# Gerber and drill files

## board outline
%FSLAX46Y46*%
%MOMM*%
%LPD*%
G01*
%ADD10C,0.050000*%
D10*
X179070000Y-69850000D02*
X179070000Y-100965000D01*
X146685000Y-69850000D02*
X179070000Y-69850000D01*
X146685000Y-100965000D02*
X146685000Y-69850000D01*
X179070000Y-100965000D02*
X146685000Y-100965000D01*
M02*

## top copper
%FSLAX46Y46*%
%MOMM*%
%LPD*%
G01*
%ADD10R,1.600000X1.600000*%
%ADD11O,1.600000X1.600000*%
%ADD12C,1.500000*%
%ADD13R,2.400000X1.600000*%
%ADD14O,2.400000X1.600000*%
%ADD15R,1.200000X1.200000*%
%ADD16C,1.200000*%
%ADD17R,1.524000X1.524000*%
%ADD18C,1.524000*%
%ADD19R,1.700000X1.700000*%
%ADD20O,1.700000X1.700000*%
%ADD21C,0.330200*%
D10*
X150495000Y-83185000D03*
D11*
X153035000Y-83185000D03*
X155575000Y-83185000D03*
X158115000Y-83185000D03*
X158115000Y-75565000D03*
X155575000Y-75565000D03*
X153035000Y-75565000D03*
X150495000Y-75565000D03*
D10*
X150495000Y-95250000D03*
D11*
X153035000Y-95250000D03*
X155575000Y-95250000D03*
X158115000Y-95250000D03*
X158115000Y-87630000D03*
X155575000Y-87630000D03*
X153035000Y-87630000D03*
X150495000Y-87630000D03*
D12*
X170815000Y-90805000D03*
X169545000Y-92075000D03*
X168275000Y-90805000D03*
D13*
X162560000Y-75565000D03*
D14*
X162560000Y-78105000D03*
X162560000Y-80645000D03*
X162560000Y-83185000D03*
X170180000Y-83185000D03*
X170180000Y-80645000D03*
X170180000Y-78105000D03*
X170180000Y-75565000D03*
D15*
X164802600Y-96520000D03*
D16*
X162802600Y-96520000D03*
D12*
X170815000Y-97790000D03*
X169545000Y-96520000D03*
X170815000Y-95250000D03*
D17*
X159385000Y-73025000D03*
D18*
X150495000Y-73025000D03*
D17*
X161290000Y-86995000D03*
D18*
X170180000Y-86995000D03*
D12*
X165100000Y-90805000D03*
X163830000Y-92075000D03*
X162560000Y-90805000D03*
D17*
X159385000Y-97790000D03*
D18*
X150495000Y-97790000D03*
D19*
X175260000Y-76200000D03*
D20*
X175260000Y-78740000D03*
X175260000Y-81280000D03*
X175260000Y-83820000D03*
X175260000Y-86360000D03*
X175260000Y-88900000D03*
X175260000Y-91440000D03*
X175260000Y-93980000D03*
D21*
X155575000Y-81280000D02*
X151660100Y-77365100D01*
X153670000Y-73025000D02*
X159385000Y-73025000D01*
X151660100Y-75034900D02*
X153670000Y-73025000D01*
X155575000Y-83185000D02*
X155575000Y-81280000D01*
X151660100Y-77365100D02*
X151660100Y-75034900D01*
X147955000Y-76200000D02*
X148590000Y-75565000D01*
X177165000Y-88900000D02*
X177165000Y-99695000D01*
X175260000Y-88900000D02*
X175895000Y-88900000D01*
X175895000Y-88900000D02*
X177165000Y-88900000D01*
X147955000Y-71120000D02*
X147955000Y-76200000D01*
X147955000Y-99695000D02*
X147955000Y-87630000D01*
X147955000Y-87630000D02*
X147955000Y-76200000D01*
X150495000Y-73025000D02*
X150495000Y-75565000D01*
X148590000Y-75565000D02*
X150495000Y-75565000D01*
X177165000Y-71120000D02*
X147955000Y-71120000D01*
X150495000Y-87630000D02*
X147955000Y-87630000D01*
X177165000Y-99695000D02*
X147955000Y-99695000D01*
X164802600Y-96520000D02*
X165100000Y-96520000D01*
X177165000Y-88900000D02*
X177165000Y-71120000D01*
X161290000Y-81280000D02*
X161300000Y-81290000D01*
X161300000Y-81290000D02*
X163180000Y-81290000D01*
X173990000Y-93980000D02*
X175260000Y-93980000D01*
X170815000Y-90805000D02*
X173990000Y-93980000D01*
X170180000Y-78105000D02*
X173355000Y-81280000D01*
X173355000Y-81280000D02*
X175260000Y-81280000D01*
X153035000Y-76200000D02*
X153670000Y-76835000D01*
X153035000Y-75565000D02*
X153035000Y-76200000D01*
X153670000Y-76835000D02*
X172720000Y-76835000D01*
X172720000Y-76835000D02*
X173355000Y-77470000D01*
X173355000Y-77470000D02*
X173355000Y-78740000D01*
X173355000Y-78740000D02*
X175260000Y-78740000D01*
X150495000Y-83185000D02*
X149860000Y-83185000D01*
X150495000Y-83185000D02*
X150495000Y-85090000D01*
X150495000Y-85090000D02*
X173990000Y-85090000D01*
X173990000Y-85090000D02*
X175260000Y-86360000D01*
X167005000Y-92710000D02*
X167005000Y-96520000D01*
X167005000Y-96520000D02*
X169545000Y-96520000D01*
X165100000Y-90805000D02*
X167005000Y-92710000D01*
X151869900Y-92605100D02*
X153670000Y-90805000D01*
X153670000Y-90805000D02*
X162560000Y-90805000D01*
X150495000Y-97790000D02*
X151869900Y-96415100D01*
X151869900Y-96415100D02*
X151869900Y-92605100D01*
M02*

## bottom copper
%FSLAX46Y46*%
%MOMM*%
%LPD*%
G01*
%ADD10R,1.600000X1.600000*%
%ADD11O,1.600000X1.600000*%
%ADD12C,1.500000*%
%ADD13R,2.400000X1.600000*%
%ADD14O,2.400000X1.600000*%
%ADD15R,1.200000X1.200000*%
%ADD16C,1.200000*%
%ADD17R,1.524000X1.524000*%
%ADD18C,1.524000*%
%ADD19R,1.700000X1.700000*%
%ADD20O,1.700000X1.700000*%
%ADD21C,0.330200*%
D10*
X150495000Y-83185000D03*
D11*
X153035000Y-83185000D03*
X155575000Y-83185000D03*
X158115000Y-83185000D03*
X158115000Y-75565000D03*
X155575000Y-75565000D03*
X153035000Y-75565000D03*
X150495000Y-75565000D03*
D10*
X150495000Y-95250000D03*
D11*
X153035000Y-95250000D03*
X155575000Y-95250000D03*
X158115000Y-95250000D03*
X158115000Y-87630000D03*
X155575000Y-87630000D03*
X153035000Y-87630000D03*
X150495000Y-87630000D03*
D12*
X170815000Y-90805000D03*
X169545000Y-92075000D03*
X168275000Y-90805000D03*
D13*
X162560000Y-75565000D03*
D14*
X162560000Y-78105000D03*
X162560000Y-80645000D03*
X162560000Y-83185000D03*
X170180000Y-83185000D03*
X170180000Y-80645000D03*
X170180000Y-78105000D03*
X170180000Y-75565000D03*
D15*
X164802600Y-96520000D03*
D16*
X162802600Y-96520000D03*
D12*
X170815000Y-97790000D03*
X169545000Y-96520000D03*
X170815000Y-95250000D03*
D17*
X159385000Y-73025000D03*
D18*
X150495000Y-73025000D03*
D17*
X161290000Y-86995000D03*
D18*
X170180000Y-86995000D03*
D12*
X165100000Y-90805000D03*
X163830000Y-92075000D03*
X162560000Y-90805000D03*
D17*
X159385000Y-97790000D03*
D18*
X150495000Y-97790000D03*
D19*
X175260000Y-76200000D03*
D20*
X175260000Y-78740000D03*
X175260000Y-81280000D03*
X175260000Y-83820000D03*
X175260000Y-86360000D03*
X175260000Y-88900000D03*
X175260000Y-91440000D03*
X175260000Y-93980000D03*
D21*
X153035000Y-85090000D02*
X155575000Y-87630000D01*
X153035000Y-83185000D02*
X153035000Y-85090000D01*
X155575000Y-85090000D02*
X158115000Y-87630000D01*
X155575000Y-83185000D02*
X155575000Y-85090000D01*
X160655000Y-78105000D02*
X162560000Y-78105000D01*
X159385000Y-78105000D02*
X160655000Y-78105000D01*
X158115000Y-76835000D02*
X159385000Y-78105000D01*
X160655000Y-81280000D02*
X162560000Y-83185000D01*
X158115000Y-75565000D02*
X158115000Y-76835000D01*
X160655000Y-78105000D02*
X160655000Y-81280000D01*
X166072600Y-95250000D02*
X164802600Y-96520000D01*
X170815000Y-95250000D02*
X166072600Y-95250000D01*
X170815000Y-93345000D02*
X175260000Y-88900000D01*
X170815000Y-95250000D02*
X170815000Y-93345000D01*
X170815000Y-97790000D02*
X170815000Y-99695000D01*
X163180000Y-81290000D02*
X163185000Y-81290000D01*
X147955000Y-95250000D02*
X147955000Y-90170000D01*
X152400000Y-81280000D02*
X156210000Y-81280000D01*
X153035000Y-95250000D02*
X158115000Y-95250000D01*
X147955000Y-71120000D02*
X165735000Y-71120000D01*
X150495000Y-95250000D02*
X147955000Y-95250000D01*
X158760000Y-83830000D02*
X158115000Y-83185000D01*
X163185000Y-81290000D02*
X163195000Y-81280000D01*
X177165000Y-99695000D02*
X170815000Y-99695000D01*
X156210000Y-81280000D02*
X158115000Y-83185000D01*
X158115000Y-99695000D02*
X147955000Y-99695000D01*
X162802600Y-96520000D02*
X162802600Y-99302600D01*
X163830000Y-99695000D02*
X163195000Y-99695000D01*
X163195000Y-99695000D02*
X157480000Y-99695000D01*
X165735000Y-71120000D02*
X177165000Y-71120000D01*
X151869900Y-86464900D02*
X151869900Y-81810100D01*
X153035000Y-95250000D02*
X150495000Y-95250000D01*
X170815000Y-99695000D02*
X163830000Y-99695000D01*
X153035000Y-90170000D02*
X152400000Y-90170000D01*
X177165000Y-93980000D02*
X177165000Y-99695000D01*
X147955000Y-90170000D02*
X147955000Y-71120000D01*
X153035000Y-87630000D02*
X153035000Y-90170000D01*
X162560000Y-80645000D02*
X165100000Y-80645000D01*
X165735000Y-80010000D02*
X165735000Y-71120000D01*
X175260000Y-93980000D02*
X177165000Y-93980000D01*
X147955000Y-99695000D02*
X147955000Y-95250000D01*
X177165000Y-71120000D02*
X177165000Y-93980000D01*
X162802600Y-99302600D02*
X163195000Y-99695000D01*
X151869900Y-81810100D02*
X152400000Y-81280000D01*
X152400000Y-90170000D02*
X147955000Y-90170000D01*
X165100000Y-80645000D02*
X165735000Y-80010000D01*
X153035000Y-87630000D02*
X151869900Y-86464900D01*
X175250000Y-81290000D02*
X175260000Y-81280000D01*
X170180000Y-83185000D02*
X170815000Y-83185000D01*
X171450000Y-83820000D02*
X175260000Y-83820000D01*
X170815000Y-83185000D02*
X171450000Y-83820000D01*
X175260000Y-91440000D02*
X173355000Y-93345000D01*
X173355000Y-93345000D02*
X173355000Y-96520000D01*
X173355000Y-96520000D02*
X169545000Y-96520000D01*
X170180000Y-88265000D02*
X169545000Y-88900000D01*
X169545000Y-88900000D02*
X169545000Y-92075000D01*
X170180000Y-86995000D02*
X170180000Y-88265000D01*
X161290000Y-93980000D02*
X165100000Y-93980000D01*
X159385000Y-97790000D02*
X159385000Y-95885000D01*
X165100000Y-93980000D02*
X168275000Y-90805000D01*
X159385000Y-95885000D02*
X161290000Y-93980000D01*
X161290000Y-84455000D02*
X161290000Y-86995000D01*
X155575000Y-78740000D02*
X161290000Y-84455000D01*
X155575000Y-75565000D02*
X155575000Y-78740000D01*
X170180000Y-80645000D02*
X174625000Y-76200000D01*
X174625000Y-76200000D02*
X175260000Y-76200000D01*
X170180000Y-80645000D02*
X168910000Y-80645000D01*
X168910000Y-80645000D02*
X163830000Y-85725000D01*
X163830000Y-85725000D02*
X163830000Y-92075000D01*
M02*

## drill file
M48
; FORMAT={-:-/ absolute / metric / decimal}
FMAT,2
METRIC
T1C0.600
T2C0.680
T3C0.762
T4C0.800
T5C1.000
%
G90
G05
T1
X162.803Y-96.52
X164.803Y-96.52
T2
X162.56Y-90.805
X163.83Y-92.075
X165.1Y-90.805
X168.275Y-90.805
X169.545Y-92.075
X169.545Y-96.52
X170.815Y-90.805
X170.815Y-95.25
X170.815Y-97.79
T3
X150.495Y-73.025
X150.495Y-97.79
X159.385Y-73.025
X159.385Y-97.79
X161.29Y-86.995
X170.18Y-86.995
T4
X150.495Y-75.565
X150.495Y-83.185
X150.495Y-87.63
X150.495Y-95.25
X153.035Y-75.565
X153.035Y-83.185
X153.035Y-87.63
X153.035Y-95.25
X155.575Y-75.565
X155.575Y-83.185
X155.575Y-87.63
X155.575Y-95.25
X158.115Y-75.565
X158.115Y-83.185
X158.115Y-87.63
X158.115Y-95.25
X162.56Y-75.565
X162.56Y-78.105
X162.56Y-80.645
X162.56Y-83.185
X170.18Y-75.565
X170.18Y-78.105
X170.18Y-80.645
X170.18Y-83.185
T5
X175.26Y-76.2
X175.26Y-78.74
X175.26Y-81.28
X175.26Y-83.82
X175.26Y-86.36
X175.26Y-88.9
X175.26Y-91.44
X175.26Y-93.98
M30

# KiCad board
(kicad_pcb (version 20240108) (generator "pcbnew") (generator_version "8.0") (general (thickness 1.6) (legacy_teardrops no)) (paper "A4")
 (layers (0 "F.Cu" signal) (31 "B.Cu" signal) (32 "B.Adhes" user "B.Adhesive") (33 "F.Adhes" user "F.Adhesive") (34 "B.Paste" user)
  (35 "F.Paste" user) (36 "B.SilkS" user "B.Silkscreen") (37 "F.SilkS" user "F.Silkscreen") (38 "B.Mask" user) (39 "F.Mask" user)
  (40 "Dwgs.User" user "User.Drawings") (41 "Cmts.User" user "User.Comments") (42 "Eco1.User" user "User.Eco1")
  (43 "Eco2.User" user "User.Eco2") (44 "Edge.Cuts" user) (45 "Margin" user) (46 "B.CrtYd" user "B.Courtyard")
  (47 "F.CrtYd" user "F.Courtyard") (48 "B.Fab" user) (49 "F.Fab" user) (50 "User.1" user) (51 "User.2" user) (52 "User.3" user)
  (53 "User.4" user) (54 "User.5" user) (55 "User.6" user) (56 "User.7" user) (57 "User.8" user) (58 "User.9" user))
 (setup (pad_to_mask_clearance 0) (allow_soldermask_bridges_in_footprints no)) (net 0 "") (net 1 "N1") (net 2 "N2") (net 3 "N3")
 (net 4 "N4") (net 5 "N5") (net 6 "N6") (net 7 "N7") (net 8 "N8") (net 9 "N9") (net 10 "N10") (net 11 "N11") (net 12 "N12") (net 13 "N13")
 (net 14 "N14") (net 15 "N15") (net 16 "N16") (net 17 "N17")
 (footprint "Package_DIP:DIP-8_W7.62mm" (layer "F.Cu") (at 150.495 83.185 90)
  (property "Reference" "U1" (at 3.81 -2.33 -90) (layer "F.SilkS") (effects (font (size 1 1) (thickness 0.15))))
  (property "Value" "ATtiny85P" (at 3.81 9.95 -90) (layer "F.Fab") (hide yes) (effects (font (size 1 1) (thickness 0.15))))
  (pad "1" thru_hole rect (at 0 0 90) (size 1.6 1.6) (drill 0.8) (layers "*.Cu" "*.Mask") (remove_unused_layers no) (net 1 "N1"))
  (pad "2" thru_hole oval (at 0 2.54 90) (size 1.6 1.6) (drill 0.8) (layers "*.Cu" "*.Mask") (remove_unused_layers no) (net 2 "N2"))
  (pad "3" thru_hole oval (at 0 5.08 90) (size 1.6 1.6) (drill 0.8) (layers "*.Cu" "*.Mask") (remove_unused_layers no) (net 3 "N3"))
  (pad "4" thru_hole oval (at 0 7.62 90) (size 1.6 1.6) (drill 0.8) (layers "*.Cu" "*.Mask") (remove_unused_layers no) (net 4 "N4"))
  (pad "5" thru_hole oval (at 7.62 7.62 90) (size 1.6 1.6) (drill 0.8) (layers "*.Cu" "*.Mask") (remove_unused_layers no) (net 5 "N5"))
  (pad "6" thru_hole oval (at 7.62 5.08 90) (size 1.6 1.6) (drill 0.8) (layers "*.Cu" "*.Mask") (remove_unused_layers no) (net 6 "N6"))
  (pad "7" thru_hole oval (at 7.62 2.54 90) (size 1.6 1.6) (drill 0.8) (layers "*.Cu" "*.Mask") (remove_unused_layers no) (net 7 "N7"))
  (pad "8" thru_hole oval (at 7.62 0 90) (size 1.6 1.6) (drill 0.8) (layers "*.Cu" "*.Mask") (remove_unused_layers no) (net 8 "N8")))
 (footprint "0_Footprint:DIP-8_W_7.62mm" (layer "F.Cu") (at 150.495 95.25 90)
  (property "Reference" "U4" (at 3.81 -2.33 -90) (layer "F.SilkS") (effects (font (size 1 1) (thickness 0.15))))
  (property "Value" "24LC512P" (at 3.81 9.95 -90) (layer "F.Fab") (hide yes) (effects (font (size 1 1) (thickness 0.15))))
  (pad "1" thru_hole rect (at 0 0 90) (size 1.6 1.6) (drill 0.8) (layers "*.Cu" "*.Mask") (remove_unused_layers no) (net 4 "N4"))
  (pad "2" thru_hole oval (at 0 2.54 90) (size 1.6 1.6) (drill 0.8) (layers "*.Cu" "*.Mask") (remove_unused_layers no) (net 4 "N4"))
  (pad "3" thru_hole oval (at 0 5.08 90) (size 1.6 1.6) (drill 0.8) (layers "*.Cu" "*.Mask") (remove_unused_layers no) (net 4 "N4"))
  (pad "4" thru_hole oval (at 0 7.62 90) (size 1.6 1.6) (drill 0.8) (layers "*.Cu" "*.Mask") (remove_unused_layers no) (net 4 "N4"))
  (pad "5" thru_hole oval (at 7.62 7.62 90) (size 1.6 1.6) (drill 0.8) (layers "*.Cu" "*.Mask") (remove_unused_layers no) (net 3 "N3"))
  (pad "6" thru_hole oval (at 7.62 5.08 90) (size 1.6 1.6) (drill 0.8) (layers "*.Cu" "*.Mask") (remove_unused_layers no) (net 2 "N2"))
  (pad "7" thru_hole oval (at 7.62 2.54 90) (size 1.6 1.6) (drill 0.8) (layers "*.Cu" "*.Mask") (remove_unused_layers no) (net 4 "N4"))
  (pad "8" thru_hole oval (at 7.62 0 90) (size 1.6 1.6) (drill 0.8) (layers "*.Cu" "*.Mask") (remove_unused_layers no) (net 8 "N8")))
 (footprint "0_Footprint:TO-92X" (layer "F.Cu") (at 170.815 90.805 180)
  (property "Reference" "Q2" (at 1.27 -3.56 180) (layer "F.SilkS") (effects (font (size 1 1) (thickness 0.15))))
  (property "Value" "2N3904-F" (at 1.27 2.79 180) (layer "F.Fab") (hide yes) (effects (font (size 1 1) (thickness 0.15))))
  (pad "1" thru_hole circle (at 0 0 180) (size 1.5 1.5) (drill 0.68) (layers "*.Cu" "*.Mask") (remove_unused_layers no) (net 4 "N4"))
  (pad "2" thru_hole circle (at 1.27 -1.27 180) (size 1.5 1.5) (drill 0.68) (layers "*.Cu" "*.Mask") (remove_unused_layers no) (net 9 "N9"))
  (pad "3" thru_hole circle (at 2.54 0 180) (size 1.5 1.5) (drill 0.68) (layers "*.Cu" "*.Mask") (remove_unused_layers no) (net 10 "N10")))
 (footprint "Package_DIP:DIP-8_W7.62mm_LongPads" (layer "F.Cu") (at 162.56 75.565)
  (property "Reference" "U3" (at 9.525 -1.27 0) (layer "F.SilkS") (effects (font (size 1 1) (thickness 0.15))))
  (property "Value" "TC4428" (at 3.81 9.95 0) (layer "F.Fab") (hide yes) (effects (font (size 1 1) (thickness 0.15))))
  (pad "1" thru_hole rect (at 0 0) (size 2.4 1.6) (drill 0.8) (layers "*.Cu" "*.Mask") (remove_unused_layers no) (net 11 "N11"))
  (pad "2" thru_hole oval (at 0 2.54) (size 2.4 1.6) (drill 0.8) (layers "*.Cu" "*.Mask") (remove_unused_layers no) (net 5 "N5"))
  (pad "3" thru_hole oval (at 0 5.08) (size 2.4 1.6) (drill 0.8) (layers "*.Cu" "*.Mask") (remove_unused_layers no) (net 4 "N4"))
  (pad "4" thru_hole oval (at 0 7.62) (size 2.4 1.6) (drill 0.8) (layers "*.Cu" "*.Mask") (remove_unused_layers no) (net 5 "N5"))
  (pad "5" thru_hole oval (at 7.62 7.62) (size 2.4 1.6) (drill 0.8) (layers "*.Cu" "*.Mask") (remove_unused_layers no) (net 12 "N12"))
  (pad "6" thru_hole oval (at 7.62 5.08) (size 2.4 1.6) (drill 0.8) (layers "*.Cu" "*.Mask") (remove_unused_layers no) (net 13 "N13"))
  (pad "7" thru_hole oval (at 7.62 2.54) (size 2.4 1.6) (drill 0.8) (layers "*.Cu" "*.Mask") (remove_unused_layers no) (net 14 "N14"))
  (pad "8" thru_hole oval (at 7.62 0) (size 2.4 1.6) (drill 0.8) (layers "*.Cu" "*.Mask") (remove_unused_layers no) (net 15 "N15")))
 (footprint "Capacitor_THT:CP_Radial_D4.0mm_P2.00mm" (layer "F.Cu") (at 164.8026 96.52 180)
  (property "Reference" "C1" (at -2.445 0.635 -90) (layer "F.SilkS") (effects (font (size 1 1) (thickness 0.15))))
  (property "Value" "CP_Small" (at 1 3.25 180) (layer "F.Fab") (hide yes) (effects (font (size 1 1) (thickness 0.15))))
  (pad "1" thru_hole rect (at 0 0 180) (size 1.2 1.2) (drill 0.6) (layers "*.Cu" "*.Mask") (remove_unused_layers no) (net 8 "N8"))
  (pad "2" thru_hole circle (at 2 0 180) (size 1.2 1.2) (drill 0.6) (layers "*.Cu" "*.Mask") (remove_unused_layers no) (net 4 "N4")))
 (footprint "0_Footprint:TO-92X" (layer "F.Cu") (at 170.815 97.79 90)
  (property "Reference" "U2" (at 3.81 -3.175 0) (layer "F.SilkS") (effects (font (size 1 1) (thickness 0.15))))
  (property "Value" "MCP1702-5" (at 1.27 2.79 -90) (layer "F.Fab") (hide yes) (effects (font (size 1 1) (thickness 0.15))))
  (pad "1" thru_hole circle (at 0 0 90) (size 1.5 1.5) (drill 0.68) (layers "*.Cu" "*.Mask") (remove_unused_layers no) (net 4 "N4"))
  (pad "2" thru_hole circle (at 1.27 -1.27 90) (size 1.5 1.5) (drill 0.68) (layers "*.Cu" "*.Mask") (remove_unused_layers no) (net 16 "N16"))
  (pad "3" thru_hole circle (at 2.54 0 90) (size 1.5 1.5) (drill 0.68) (layers "*.Cu" "*.Mask") (remove_unused_layers no) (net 8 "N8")))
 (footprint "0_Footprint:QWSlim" (layer "F.Cu") (at 159.385 73.025 180)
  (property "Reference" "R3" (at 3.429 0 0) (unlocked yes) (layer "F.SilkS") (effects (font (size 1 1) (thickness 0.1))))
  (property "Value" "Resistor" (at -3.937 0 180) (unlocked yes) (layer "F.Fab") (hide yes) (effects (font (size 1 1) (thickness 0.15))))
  (pad "1" thru_hole rect (at 0 0 180) (size 1.524 1.524) (drill 0.762) (layers "*.Cu" "*.Mask") (remove_unused_layers no) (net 3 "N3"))
  (pad "2" thru_hole circle (at 8.89 0 180) (size 1.524 1.524) (drill 0.762) (layers "*.Cu" "*.Mask") (remove_unused_layers no) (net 8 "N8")))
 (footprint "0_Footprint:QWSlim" (layer "F.Cu") (at 161.29 86.995)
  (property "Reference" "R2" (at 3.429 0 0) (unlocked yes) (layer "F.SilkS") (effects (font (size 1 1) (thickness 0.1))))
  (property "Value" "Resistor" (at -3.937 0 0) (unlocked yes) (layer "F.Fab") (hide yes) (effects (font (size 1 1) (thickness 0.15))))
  (pad "1" thru_hole rect (at 0 0) (size 1.524 1.524) (drill 0.762) (layers "*.Cu" "*.Mask") (remove_unused_layers no) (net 6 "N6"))
  (pad "2" thru_hole circle (at 8.89 0) (size 1.524 1.524) (drill 0.762) (layers "*.Cu" "*.Mask") (remove_unused_layers no) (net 9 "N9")))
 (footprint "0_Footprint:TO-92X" (layer "F.Cu") (at 165.1 90.805 180)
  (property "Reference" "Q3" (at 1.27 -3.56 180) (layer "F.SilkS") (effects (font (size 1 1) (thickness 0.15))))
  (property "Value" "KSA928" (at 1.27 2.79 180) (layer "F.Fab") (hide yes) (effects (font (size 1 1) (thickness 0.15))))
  (pad "1" thru_hole circle (at 0 0 180) (size 1.5 1.5) (drill 0.68) (layers "*.Cu" "*.Mask") (remove_unused_layers no) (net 16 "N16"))
  (pad "2" thru_hole circle (at 1.27 -1.27 180) (size 1.5 1.5) (drill 0.68) (layers "*.Cu" "*.Mask") (remove_unused_layers no)
   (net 13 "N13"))
  (pad "3" thru_hole circle (at 2.54 0 180) (size 1.5 1.5) (drill 0.68) (layers "*.Cu" "*.Mask") (remove_unused_layers no) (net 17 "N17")))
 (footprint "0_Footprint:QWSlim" (layer "F.Cu") (at 159.385 97.79 180)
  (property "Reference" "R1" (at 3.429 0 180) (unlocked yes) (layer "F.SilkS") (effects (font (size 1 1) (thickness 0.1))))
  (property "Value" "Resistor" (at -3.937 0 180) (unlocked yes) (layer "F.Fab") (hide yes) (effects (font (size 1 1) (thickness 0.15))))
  (pad "1" thru_hole rect (at 0 0 180) (size 1.524 1.524) (drill 0.762) (layers "*.Cu" "*.Mask") (remove_unused_layers no) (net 10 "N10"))
  (pad "2" thru_hole circle (at 8.89 0 180) (size 1.524 1.524) (drill 0.762) (layers "*.Cu" "*.Mask") (remove_unused_layers no)
   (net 17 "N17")))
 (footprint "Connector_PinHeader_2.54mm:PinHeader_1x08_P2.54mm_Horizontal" (layer "F.Cu") (at 175.26 76.2)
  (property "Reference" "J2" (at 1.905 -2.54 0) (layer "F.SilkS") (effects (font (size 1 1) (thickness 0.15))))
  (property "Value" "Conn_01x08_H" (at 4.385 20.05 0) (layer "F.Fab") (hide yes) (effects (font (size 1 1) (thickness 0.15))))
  (pad "1" thru_hole rect (at 0 0) (size 1.7 1.7) (drill 1) (layers "*.Cu" "*.Mask") (remove_unused_layers no) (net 13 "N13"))
  (pad "2" thru_hole oval (at 0 2.54) (size 1.7 1.7) (drill 1) (layers "*.Cu" "*.Mask") (remove_unused_layers no) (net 7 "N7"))
  (pad "3" thru_hole oval (at 0 5.08) (size 1.7 1.7) (drill 1) (layers "*.Cu" "*.Mask") (remove_unused_layers no) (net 14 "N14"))
  (pad "4" thru_hole oval (at 0 7.62) (size 1.7 1.7) (drill 1) (layers "*.Cu" "*.Mask") (remove_unused_layers no) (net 12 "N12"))
  (pad "5" thru_hole oval (at 0 10.16) (size 1.7 1.7) (drill 1) (layers "*.Cu" "*.Mask") (remove_unused_layers no) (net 1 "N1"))
  (pad "6" thru_hole oval (at 0 12.7) (size 1.7 1.7) (drill 1) (layers "*.Cu" "*.Mask") (remove_unused_layers no) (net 8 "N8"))
  (pad "7" thru_hole oval (at 0 15.24) (size 1.7 1.7) (drill 1) (layers "*.Cu" "*.Mask") (remove_unused_layers no) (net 16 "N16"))
  (pad "8" thru_hole oval (at 0 17.78) (size 1.7 1.7) (drill 1) (layers "*.Cu" "*.Mask") (remove_unused_layers no) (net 4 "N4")))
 (gr_line (start 179.07 69.85) (end 179.07 100.965) (stroke (width 0.05) (type default)) (layer "Edge.Cuts"))
 (gr_line (start 146.685 69.85) (end 179.07 69.85) (stroke (width 0.05) (type default)) (layer "Edge.Cuts"))
 (gr_line (start 146.685 100.965) (end 146.685 69.85) (stroke (width 0.05) (type default)) (layer "Edge.Cuts"))
 (gr_line (start 179.07 100.965) (end 146.685 100.965) (stroke (width 0.05) (type default)) (layer "Edge.Cuts"))
 (segment (start 153.035 85.09) (end 155.575 87.63) (width 0.3302) (layer "B.Cu") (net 2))
 (segment (start 153.035 83.185) (end 153.035 85.09) (width 0.3302) (layer "B.Cu") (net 2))
 (segment (start 155.575 81.28) (end 151.6601 77.3651) (width 0.3302) (layer "F.Cu") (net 3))
 (segment (start 153.67 73.025) (end 159.385 73.025) (width 0.3302) (layer "F.Cu") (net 3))
 (segment (start 151.6601 75.0349) (end 153.67 73.025) (width 0.3302) (layer "F.Cu") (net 3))
 (segment (start 155.575 83.185) (end 155.575 81.28) (width 0.3302) (layer "F.Cu") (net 3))
 (segment (start 151.6601 77.3651) (end 151.6601 75.0349) (width 0.3302) (layer "F.Cu") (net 3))
 (segment (start 155.575 85.09) (end 158.115 87.63) (width 0.3302) (layer "B.Cu") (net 3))
 (segment (start 155.575 83.185) (end 155.575 85.09) (width 0.3302) (layer "B.Cu") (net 3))
 (segment (start 160.655 78.105) (end 162.56 78.105) (width 0.3302) (layer "B.Cu") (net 5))
 (segment (start 159.385 78.105) (end 160.655 78.105) (width 0.3302) (layer "B.Cu") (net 5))
 (segment (start 158.115 76.835) (end 159.385 78.105) (width 0.3302) (layer "B.Cu") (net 5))
 (segment (start 160.655 81.28) (end 162.56 83.185) (width 0.3302) (layer "B.Cu") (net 5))
 (segment (start 158.115 75.565) (end 158.115 76.835) (width 0.3302) (layer "B.Cu") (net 5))
 (segment (start 160.655 78.105) (end 160.655 81.28) (width 0.3302) (layer "B.Cu") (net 5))
 (segment (start 147.955 76.2) (end 148.59 75.565) (width 0.3302) (layer "F.Cu") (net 8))
 (segment (start 177.165 88.9) (end 177.165 99.695) (width 0.3302) (layer "F.Cu") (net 8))
 (segment (start 175.26 88.9) (end 175.895 88.9) (width 0.3302) (layer "F.Cu") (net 8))
 (segment (start 175.895 88.9) (end 177.165 88.9) (width 0.3302) (layer "F.Cu") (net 8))
 (segment (start 147.955 71.12) (end 147.955 76.2) (width 0.3302) (layer "F.Cu") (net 8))
 (segment (start 147.955 99.695) (end 147.955 87.63) (width 0.3302) (layer "F.Cu") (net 8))
 (segment (start 147.955 87.63) (end 147.955 76.2) (width 0.3302) (layer "F.Cu") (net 8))
 (segment (start 150.495 73.025) (end 150.495 75.565) (width 0.3302) (layer "F.Cu") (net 8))
 (segment (start 148.59 75.565) (end 150.495 75.565) (width 0.3302) (layer "F.Cu") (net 8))
 (segment (start 177.165 71.12) (end 147.955 71.12) (width 0.3302) (layer "F.Cu") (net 8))
 (segment (start 150.495 87.63) (end 147.955 87.63) (width 0.3302) (layer "F.Cu") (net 8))
 (segment (start 177.165 99.695) (end 147.955 99.695) (width 0.3302) (layer "F.Cu") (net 8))
 (segment (start 164.8026 96.52) (end 165.1 96.52) (width 0.3302) (layer "F.Cu") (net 8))
 (segment (start 177.165 88.9) (end 177.165 71.12) (width 0.3302) (layer "F.Cu") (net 8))
 (segment (start 166.0726 95.25) (end 164.8026 96.52) (width 0.3302) (layer "B.Cu") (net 8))
 (segment (start 170.815 95.25) (end 166.0726 95.25) (width 0.3302) (layer "B.Cu") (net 8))
 (segment (start 170.815 93.345) (end 175.26 88.9) (width 0.3302) (layer "B.Cu") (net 8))
 (segment (start 170.815 95.25) (end 170.815 93.345) (width 0.3302) (layer "B.Cu") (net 8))
 (segment (start 161.29 81.28) (end 161.3 81.29) (width 0.3302) (layer "F.Cu") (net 4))
 (segment (start 161.3 81.29) (end 163.18 81.29) (width 0.3302) (layer "F.Cu") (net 4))
 (segment (start 173.99 93.98) (end 175.26 93.98) (width 0.3302) (layer "F.Cu") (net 4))
 (segment (start 170.815 90.805) (end 173.99 93.98) (width 0.3302) (layer "F.Cu") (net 4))
 (segment (start 170.815 97.79) (end 170.815 99.695) (width 0.3302) (layer "B.Cu") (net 4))
 (segment (start 163.18 81.29) (end 163.185 81.29) (width 0.3302) (layer "B.Cu") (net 4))
 (segment (start 147.955 95.25) (end 147.955 90.17) (width 0.3302) (layer "B.Cu") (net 4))
 (segment (start 152.4 81.28) (end 156.21 81.28) (width 0.3302) (layer "B.Cu") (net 4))
 (segment (start 153.035 95.25) (end 158.115 95.25) (width 0.3302) (layer "B.Cu") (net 4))
 (segment (start 147.955 71.12) (end 165.735 71.12) (width 0.3302) (layer "B.Cu") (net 4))
 (segment (start 150.495 95.25) (end 147.955 95.25) (width 0.3302) (layer "B.Cu") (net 4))
 (segment (start 158.76 83.83) (end 158.115 83.185) (width 0.3302) (layer "B.Cu") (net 4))
 (segment (start 163.185 81.29) (end 163.195 81.28) (width 0.3302) (layer "B.Cu") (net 4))
 (segment (start 177.165 99.695) (end 170.815 99.695) (width 0.3302) (layer "B.Cu") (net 4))
 (segment (start 156.21 81.28) (end 158.115 83.185) (width 0.3302) (layer "B.Cu") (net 4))
 (segment (start 158.115 99.695) (end 147.955 99.695) (width 0.3302) (layer "B.Cu") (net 4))
 (segment (start 162.8026 96.52) (end 162.8026 99.3026) (width 0.3302) (layer "B.Cu") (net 4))
 (segment (start 163.83 99.695) (end 163.195 99.695) (width 0.3302) (layer "B.Cu") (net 4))
 (segment (start 163.195 99.695) (end 157.48 99.695) (width 0.3302) (layer "B.Cu") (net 4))
 (segment (start 165.735 71.12) (end 177.165 71.12) (width 0.3302) (layer "B.Cu") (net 4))
 (segment (start 151.8699 86.4649) (end 151.8699 81.8101) (width 0.3302) (layer "B.Cu") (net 4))
 (segment (start 153.035 95.25) (end 150.495 95.25) (width 0.3302) (layer "B.Cu") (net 4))
 (segment (start 170.815 99.695) (end 163.83 99.695) (width 0.3302) (layer "B.Cu") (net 4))
 (segment (start 153.035 90.17) (end 152.4 90.17) (width 0.3302) (layer "B.Cu") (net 4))
 (segment (start 177.165 93.98) (end 177.165 99.695) (width 0.3302) (layer "B.Cu") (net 4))
 (segment (start 147.955 90.17) (end 147.955 71.12) (width 0.3302) (layer "B.Cu") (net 4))
 (segment (start 153.035 87.63) (end 153.035 90.17) (width 0.3302) (layer "B.Cu") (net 4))
 (segment (start 162.56 80.645) (end 165.1 80.645) (width 0.3302) (layer "B.Cu") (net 4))
 (segment (start 165.735 80.01) (end 165.735 71.12) (width 0.3302) (layer "B.Cu") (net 4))
 (segment (start 175.26 93.98) (end 177.165 93.98) (width 0.3302) (layer "B.Cu") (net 4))
 (segment (start 147.955 99.695) (end 147.955 95.25) (width 0.3302) (layer "B.Cu") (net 4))
 (segment (start 177.165 71.12) (end 177.165 93.98) (width 0.3302) (layer "B.Cu") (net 4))
 (segment (start 162.8026 99.3026) (end 163.195 99.695) (width 0.3302) (layer "B.Cu") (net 4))
 (segment (start 151.8699 81.8101) (end 152.4 81.28) (width 0.3302) (layer "B.Cu") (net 4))
 (segment (start 152.4 90.17) (end 147.955 90.17) (width 0.3302) (layer "B.Cu") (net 4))
 (segment (start 165.1 80.645) (end 165.735 80.01) (width 0.3302) (layer "B.Cu") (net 4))
 (segment (start 153.035 87.63) (end 151.8699 86.4649) (width 0.3302) (layer "B.Cu") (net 4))
 (segment (start 170.18 78.105) (end 173.355 81.28) (width 0.3302) (layer "F.Cu") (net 14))
 (segment (start 173.355 81.28) (end 175.26 81.28) (width 0.3302) (layer "F.Cu") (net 14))
 (segment (start 175.25 81.29) (end 175.26 81.28) (width 0.3302) (layer "B.Cu") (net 14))
 (segment (start 153.035 76.2) (end 153.67 76.835) (width 0.3302) (layer "F.Cu") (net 7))
 (segment (start 153.035 75.565) (end 153.035 76.2) (width 0.3302) (layer "F.Cu") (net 7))
 (segment (start 153.67 76.835) (end 172.72 76.835) (width 0.3302) (layer "F.Cu") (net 7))
 (segment (start 172.72 76.835) (end 173.355 77.47) (width 0.3302) (layer "F.Cu") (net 7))
 (segment (start 173.355 77.47) (end 173.355 78.74) (width 0.3302) (layer "F.Cu") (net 7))
 (segment (start 173.355 78.74) (end 175.26 78.74) (width 0.3302) (layer "F.Cu") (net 7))
 (segment (start 150.495 83.185) (end 149.86 83.185) (width 0.3302) (layer "F.Cu") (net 1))
 (segment (start 150.495 83.185) (end 150.495 85.09) (width 0.3302) (layer "F.Cu") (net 1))
 (segment (start 150.495 85.09) (end 173.99 85.09) (width 0.3302) (layer "F.Cu") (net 1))
 (segment (start 173.99 85.09) (end 175.26 86.36) (width 0.3302) (layer "F.Cu") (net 1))
 (segment (start 170.18 83.185) (end 170.815 83.185) (width 0.3302) (layer "B.Cu") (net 12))
 (segment (start 171.45 83.82) (end 175.26 83.82) (width 0.3302) (layer "B.Cu") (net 12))
 (segment (start 170.815 83.185) (end 171.45 83.82) (width 0.3302) (layer "B.Cu") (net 12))
 (segment (start 167.005 92.71) (end 167.005 96.52) (width 0.3302) (layer "F.Cu") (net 16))
 (segment (start 167.005 96.52) (end 169.545 96.52) (width 0.3302) (layer "F.Cu") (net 16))
 (segment (start 165.1 90.805) (end 167.005 92.71) (width 0.3302) (layer "F.Cu") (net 16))
 (segment (start 175.26 91.44) (end 173.355 93.345) (width 0.3302) (layer "B.Cu") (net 16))
 (segment (start 173.355 93.345) (end 173.355 96.52) (width 0.3302) (layer "B.Cu") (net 16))
 (segment (start 173.355 96.52) (end 169.545 96.52) (width 0.3302) (layer "B.Cu") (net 16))
 (segment (start 170.18 88.265) (end 169.545 88.9) (width 0.3302) (layer "B.Cu") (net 9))
 (segment (start 169.545 88.9) (end 169.545 92.075) (width 0.3302) (layer "B.Cu") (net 9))
 (segment (start 170.18 86.995) (end 170.18 88.265) (width 0.3302) (layer "B.Cu") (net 9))
 (segment (start 161.29 93.98) (end 165.1 93.98) (width 0.3302) (layer "B.Cu") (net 10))
 (segment (start 159.385 97.79) (end 159.385 95.885) (width 0.3302) (layer "B.Cu") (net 10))
 (segment (start 165.1 93.98) (end 168.275 90.805) (width 0.3302) (layer "B.Cu") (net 10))
 (segment (start 159.385 95.885) (end 161.29 93.98) (width 0.3302) (layer "B.Cu") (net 10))
 (segment (start 151.8699 92.6051) (end 153.67 90.805) (width 0.3302) (layer "F.Cu") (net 17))
 (segment (start 153.67 90.805) (end 162.56 90.805) (width 0.3302) (layer "F.Cu") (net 17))
 (segment (start 150.495 97.79) (end 151.8699 96.4151) (width 0.3302) (layer "F.Cu") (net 17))
 (segment (start 151.8699 96.4151) (end 151.8699 92.6051) (width 0.3302) (layer "F.Cu") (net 17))
 (segment (start 161.29 84.455) (end 161.29 86.995) (width 0.3302) (layer "B.Cu") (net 6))
 (segment (start 155.575 78.74) (end 161.29 84.455) (width 0.3302) (layer "B.Cu") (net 6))
 (segment (start 155.575 75.565) (end 155.575 78.74) (width 0.3302) (layer "B.Cu") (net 6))
 (segment (start 170.18 80.645) (end 174.625 76.2) (width 0.3302) (layer "B.Cu") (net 13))
 (segment (start 174.625 76.2) (end 175.26 76.2) (width 0.3302) (layer "B.Cu") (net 13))
 (segment (start 170.18 80.645) (end 168.91 80.645) (width 0.3302) (layer "B.Cu") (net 13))
 (segment (start 168.91 80.645) (end 163.83 85.725) (width 0.3302) (layer "B.Cu") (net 13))
 (segment (start 163.83 85.725) (end 163.83 92.075) (width 0.3302) (layer "B.Cu") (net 13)))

